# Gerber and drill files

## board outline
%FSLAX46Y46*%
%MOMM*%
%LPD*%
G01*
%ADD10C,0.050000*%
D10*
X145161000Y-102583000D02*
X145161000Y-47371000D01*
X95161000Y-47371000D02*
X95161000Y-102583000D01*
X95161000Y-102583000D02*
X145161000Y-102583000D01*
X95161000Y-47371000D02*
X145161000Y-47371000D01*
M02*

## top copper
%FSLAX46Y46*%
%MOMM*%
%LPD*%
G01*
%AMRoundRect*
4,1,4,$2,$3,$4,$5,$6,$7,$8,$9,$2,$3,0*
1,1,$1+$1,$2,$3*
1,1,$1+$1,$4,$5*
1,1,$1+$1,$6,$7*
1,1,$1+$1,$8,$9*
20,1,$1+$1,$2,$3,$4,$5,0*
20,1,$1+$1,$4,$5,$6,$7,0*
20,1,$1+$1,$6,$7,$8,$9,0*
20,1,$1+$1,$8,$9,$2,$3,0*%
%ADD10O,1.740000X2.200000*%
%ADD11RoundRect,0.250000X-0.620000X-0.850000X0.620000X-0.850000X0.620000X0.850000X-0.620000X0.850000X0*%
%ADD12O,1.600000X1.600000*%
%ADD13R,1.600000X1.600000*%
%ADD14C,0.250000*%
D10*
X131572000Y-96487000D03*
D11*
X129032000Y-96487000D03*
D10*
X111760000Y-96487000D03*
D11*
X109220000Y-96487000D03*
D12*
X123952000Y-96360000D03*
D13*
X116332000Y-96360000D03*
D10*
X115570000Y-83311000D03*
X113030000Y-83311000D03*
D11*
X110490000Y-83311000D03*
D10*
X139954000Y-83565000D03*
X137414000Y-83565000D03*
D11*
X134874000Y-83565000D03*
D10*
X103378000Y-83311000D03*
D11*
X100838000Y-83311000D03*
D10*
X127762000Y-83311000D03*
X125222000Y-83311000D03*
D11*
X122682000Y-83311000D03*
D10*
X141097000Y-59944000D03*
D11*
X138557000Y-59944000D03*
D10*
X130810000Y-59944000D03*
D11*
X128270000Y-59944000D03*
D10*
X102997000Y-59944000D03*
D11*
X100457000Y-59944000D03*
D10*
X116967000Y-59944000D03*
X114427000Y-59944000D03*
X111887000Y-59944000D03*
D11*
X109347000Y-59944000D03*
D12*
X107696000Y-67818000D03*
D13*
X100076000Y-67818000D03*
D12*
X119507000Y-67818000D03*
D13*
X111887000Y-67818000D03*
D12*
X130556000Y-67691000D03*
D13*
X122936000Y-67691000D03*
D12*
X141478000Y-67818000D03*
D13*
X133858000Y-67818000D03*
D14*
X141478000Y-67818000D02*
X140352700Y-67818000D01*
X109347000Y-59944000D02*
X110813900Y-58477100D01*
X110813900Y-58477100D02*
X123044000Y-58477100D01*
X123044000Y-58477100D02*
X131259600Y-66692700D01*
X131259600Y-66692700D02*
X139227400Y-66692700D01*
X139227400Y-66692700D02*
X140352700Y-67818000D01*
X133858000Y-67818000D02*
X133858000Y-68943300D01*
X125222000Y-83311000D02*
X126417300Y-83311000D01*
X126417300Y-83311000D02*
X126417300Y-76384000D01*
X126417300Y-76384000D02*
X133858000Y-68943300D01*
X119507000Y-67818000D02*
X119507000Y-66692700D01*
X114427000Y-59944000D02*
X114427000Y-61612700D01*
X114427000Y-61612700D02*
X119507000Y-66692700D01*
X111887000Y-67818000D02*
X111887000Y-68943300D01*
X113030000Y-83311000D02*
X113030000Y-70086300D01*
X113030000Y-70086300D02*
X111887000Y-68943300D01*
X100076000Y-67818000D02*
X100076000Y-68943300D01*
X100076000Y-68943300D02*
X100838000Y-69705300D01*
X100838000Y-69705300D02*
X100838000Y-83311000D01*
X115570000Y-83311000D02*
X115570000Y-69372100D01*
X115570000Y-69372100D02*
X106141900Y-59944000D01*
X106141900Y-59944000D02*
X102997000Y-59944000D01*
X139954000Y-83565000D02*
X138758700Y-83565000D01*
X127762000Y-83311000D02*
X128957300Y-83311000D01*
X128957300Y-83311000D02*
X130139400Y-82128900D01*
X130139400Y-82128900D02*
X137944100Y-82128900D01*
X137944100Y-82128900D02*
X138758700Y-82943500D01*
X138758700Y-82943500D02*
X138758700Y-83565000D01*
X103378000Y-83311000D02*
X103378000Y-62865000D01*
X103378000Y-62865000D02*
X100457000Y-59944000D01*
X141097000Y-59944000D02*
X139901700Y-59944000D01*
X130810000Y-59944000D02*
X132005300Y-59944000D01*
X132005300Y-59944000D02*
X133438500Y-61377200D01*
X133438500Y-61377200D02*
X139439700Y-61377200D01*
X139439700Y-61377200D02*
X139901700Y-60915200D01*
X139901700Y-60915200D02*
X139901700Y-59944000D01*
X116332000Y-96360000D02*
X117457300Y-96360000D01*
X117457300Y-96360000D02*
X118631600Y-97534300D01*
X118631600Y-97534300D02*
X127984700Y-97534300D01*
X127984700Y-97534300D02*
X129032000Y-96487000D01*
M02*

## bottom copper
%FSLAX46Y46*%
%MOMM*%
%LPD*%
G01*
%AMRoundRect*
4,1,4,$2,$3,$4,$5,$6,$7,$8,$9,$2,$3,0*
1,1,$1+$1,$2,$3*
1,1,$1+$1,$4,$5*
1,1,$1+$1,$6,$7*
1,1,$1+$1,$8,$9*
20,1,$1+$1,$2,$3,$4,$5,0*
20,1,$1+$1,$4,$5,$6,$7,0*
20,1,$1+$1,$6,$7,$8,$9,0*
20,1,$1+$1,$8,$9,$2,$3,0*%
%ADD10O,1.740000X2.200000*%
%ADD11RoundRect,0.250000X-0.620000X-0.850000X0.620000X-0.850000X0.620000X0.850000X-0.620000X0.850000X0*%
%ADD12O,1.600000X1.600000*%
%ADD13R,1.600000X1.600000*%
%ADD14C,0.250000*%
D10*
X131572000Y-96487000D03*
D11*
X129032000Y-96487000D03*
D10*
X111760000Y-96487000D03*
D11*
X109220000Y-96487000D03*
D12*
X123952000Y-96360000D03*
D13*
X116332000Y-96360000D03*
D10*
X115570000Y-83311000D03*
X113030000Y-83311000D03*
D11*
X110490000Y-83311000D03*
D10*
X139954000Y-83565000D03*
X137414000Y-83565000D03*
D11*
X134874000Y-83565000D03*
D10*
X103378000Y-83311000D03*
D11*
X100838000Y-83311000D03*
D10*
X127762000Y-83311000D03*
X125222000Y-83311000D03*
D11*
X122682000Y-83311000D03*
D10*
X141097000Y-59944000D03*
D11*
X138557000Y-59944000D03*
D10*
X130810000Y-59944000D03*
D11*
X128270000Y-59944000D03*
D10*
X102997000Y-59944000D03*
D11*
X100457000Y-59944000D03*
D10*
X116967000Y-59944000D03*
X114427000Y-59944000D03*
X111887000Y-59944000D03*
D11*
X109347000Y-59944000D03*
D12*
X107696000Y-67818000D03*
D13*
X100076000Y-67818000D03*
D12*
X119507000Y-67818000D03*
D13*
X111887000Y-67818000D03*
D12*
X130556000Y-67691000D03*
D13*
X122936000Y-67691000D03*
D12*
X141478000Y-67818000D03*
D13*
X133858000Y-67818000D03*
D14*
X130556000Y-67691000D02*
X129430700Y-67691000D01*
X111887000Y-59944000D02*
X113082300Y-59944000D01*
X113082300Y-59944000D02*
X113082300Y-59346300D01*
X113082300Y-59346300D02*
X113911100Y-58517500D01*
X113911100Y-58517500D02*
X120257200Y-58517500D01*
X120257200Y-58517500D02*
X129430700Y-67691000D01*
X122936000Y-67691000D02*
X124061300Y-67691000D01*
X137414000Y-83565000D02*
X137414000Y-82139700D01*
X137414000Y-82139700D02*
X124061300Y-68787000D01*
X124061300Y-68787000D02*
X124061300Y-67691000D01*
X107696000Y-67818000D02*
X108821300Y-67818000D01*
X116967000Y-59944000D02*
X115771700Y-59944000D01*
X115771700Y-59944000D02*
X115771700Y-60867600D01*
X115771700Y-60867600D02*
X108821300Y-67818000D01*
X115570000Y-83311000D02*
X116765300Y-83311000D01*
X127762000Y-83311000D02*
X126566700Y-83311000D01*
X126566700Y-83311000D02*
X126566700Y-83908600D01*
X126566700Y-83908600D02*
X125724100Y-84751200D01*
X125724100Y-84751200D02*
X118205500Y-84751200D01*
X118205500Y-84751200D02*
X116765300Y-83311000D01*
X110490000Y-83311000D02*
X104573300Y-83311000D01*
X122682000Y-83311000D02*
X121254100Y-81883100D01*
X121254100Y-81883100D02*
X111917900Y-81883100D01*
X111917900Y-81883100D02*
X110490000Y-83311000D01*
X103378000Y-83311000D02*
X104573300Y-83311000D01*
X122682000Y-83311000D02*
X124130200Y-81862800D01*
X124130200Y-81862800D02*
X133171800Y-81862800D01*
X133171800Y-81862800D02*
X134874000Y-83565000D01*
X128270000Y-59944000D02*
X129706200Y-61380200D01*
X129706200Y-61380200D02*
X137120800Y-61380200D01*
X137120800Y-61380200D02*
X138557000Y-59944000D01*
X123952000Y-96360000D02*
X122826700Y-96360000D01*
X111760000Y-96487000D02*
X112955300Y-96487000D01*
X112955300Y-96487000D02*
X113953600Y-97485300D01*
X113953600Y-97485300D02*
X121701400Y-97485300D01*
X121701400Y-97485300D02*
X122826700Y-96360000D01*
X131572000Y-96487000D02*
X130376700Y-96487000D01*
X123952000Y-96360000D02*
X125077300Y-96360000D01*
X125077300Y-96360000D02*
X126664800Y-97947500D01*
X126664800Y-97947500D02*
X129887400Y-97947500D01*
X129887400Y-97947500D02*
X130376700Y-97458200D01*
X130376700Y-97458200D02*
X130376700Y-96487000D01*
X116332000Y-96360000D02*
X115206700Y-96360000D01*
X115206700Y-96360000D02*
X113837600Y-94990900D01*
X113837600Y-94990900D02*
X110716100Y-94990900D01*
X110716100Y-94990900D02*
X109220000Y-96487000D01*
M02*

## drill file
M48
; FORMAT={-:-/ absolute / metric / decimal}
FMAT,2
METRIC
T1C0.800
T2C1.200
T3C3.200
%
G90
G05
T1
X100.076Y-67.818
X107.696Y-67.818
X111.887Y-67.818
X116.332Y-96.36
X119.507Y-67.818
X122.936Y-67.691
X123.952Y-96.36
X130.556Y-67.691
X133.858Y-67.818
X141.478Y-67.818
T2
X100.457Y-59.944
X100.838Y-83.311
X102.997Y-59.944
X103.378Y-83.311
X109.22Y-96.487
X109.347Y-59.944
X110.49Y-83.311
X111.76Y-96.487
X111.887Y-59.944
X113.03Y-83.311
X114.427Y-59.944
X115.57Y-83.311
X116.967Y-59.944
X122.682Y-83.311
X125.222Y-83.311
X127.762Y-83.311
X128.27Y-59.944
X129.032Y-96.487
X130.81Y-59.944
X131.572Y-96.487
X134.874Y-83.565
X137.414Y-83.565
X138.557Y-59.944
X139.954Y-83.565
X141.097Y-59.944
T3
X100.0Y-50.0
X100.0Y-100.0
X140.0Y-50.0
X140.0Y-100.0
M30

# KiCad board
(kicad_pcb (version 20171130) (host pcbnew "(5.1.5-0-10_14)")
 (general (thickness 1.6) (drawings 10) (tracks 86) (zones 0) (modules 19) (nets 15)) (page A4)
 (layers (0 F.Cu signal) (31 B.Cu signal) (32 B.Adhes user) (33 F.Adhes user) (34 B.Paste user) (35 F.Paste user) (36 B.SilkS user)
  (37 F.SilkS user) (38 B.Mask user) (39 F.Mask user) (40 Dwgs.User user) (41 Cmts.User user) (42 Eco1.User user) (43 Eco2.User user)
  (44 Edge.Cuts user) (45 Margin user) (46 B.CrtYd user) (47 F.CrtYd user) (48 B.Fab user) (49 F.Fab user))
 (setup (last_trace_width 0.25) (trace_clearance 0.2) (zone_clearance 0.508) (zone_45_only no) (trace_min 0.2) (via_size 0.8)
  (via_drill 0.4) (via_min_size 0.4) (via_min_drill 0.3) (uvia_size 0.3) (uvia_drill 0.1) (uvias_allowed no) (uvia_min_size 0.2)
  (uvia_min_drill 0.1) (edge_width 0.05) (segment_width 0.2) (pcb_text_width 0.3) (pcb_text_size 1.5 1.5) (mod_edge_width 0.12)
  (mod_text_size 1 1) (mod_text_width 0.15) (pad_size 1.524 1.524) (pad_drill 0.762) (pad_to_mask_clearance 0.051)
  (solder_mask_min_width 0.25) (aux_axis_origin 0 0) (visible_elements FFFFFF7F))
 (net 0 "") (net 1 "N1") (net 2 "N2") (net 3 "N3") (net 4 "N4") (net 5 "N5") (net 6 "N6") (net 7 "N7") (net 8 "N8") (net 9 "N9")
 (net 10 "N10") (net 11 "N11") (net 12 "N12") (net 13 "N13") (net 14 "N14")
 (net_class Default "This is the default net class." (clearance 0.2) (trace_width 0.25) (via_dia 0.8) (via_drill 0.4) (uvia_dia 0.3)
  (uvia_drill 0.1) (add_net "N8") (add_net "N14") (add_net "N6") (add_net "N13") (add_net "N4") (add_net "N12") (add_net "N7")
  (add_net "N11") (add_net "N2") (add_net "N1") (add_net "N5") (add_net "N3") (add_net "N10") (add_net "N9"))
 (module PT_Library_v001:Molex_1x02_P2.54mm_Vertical (layer F.Cu) (at 129.032 96.487)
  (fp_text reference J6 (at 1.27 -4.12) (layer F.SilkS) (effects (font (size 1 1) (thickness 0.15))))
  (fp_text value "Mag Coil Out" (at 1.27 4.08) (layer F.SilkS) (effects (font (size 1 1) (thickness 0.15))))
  (pad 2 thru_hole oval (at 2.54 0) (size 1.74 2.2) (drill 1.2) (layers *.Cu *.Mask) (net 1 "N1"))
  (pad 1 thru_hole roundrect (at 0 0) (size 1.74 2.2) (drill 1.2) (layers *.Cu *.Mask) (roundrect_rratio 0.143678) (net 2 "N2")))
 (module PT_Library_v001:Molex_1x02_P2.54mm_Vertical (layer F.Cu) (at 109.22 96.487)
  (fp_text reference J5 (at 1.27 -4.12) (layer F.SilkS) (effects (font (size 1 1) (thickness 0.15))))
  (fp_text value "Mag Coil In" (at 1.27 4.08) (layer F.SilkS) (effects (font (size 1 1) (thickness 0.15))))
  (pad 2 thru_hole oval (at 2.54 0) (size 1.74 2.2) (drill 1.2) (layers *.Cu *.Mask) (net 1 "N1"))
  (pad 1 thru_hole roundrect (at 0 0) (size 1.74 2.2) (drill 1.2) (layers *.Cu *.Mask) (roundrect_rratio 0.143678) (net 2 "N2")))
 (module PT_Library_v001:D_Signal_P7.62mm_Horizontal (layer F.Cu) (at 116.332 96.36)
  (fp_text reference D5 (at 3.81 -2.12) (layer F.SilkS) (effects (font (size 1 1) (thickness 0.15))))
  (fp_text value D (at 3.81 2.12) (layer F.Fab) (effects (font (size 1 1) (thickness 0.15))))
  (pad 2 thru_hole oval (at 7.62 0) (size 1.6 1.6) (drill 0.8) (layers *.Cu *.Mask) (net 1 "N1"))
  (pad 1 thru_hole rect (at 0 0) (size 1.6 1.6) (drill 0.8) (layers *.Cu *.Mask) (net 2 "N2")))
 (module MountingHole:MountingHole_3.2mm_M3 (layer F.Cu) (at 140 100)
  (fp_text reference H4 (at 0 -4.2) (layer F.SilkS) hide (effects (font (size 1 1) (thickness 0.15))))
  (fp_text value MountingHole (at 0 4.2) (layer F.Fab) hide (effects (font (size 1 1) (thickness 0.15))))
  (pad 1 np_thru_hole circle (at 0 0) (size 3.2 3.2) (drill 3.2) (layers *.Cu *.Mask)))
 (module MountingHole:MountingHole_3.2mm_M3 (layer F.Cu) (at 100 100)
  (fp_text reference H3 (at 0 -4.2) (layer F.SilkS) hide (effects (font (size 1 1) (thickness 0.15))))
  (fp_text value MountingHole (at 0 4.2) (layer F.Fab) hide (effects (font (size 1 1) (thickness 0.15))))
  (pad 1 np_thru_hole circle (at 0 0) (size 3.2 3.2) (drill 3.2) (layers *.Cu *.Mask)))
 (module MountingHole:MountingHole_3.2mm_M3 (layer F.Cu) (at 140 50)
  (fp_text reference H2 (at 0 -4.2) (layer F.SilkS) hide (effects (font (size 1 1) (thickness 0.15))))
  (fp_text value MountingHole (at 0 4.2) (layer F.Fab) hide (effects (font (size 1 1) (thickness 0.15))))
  (pad 1 np_thru_hole circle (at 0 0) (size 3.2 3.2) (drill 3.2) (layers *.Cu *.Mask)))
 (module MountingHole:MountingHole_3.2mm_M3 (layer F.Cu) (at 100 50)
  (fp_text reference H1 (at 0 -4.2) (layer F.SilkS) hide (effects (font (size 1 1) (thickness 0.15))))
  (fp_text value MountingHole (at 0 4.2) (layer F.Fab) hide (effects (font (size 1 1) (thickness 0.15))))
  (pad 1 np_thru_hole circle (at 0 0) (size 3.2 3.2) (drill 3.2) (layers *.Cu *.Mask)))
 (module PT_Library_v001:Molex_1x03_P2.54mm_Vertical (layer F.Cu) (at 110.49 83.311)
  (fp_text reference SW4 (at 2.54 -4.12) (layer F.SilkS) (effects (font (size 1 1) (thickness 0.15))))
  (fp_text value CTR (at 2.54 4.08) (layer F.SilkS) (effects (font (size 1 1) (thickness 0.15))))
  (pad 3 thru_hole oval (at 5.08 0) (size 1.74 2.2) (drill 1.2) (layers *.Cu *.Mask) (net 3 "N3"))
  (pad 2 thru_hole oval (at 2.54 0) (size 1.74 2.2) (drill 1.2) (layers *.Cu *.Mask) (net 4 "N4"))
  (pad 1 thru_hole roundrect (at 0 0) (size 1.74 2.2) (drill 1.2) (layers *.Cu *.Mask) (roundrect_rratio 0.143678) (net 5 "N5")))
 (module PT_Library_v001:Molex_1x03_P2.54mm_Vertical (layer F.Cu) (at 134.874 83.565)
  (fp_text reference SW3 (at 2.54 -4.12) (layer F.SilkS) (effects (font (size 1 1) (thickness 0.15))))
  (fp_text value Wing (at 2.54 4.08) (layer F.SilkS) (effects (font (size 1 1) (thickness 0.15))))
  (pad 3 thru_hole oval (at 5.08 0) (size 1.74 2.2) (drill 1.2) (layers *.Cu *.Mask) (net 3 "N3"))
  (pad 2 thru_hole oval (at 2.54 0) (size 1.74 2.2) (drill 1.2) (layers *.Cu *.Mask) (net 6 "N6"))
  (pad 1 thru_hole roundrect (at 0 0) (size 1.74 2.2) (drill 1.2) (layers *.Cu *.Mask) (roundrect_rratio 0.143678) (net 5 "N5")))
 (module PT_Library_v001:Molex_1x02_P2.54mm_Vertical (layer F.Cu) (at 100.838 83.311)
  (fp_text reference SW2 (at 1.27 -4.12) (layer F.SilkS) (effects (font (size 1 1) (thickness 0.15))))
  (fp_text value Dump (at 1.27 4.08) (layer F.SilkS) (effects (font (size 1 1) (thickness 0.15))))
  (pad 2 thru_hole oval (at 2.54 0) (size 1.74 2.2) (drill 1.2) (layers *.Cu *.Mask) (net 5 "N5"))
  (pad 1 thru_hole roundrect (at 0 0) (size 1.74 2.2) (drill 1.2) (layers *.Cu *.Mask) (roundrect_rratio 0.143678) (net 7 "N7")))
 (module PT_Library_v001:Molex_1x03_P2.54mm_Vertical (layer F.Cu) (at 122.682 83.311)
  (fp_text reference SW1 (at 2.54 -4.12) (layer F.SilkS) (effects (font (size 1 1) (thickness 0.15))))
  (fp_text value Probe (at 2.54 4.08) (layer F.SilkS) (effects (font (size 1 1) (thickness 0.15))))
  (pad 3 thru_hole oval (at 5.08 0) (size 1.74 2.2) (drill 1.2) (layers *.Cu *.Mask) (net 3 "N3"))
  (pad 2 thru_hole oval (at 2.54 0) (size 1.74 2.2) (drill 1.2) (layers *.Cu *.Mask) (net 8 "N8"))
  (pad 1 thru_hole roundrect (at 0 0) (size 1.74 2.2) (drill 1.2) (layers *.Cu *.Mask) (roundrect_rratio 0.143678) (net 5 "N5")))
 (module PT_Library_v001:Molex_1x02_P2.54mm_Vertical (layer F.Cu) (at 138.557 59.944)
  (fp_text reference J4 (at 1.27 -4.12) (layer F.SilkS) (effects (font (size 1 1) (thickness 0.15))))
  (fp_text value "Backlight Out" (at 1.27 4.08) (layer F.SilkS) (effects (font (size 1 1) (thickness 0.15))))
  (pad 2 thru_hole oval (at 2.54 0) (size 1.74 2.2) (drill 1.2) (layers *.Cu *.Mask) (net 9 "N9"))
  (pad 1 thru_hole roundrect (at 0 0) (size 1.74 2.2) (drill 1.2) (layers *.Cu *.Mask) (roundrect_rratio 0.143678) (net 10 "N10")))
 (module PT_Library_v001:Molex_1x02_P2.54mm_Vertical (layer F.Cu) (at 128.27 59.944)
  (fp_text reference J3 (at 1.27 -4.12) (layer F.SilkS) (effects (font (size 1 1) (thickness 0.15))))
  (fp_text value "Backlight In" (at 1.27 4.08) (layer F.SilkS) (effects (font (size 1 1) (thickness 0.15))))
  (pad 2 thru_hole oval (at 2.54 0) (size 1.74 2.2) (drill 1.2) (layers *.Cu *.Mask) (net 9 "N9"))
  (pad 1 thru_hole roundrect (at 0 0) (size 1.74 2.2) (drill 1.2) (layers *.Cu *.Mask) (roundrect_rratio 0.143678) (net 10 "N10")))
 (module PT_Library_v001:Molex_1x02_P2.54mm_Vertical (layer F.Cu) (at 100.457 59.944)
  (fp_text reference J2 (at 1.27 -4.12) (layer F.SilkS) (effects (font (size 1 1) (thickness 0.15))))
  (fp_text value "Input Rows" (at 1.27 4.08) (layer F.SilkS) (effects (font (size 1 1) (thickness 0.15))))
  (pad 2 thru_hole oval (at 2.54 0) (size 1.74 2.2) (drill 1.2) (layers *.Cu *.Mask) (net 3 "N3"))
  (pad 1 thru_hole roundrect (at 0 0) (size 1.74 2.2) (drill 1.2) (layers *.Cu *.Mask) (roundrect_rratio 0.143678) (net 5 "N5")))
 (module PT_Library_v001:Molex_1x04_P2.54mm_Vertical (layer F.Cu) (at 109.347 59.944)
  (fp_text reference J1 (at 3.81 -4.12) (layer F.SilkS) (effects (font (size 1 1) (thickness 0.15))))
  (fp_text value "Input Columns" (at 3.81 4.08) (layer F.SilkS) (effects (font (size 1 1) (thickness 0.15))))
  (pad 4 thru_hole oval (at 7.62 0) (size 1.74 2.2) (drill 1.2) (layers *.Cu *.Mask) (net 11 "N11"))
  (pad 3 thru_hole oval (at 5.08 0) (size 1.74 2.2) (drill 1.2) (layers *.Cu *.Mask) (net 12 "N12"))
  (pad 2 thru_hole oval (at 2.54 0) (size 1.74 2.2) (drill 1.2) (layers *.Cu *.Mask) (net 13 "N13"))
  (pad 1 thru_hole roundrect (at 0 0) (size 1.74 2.2) (drill 1.2) (layers *.Cu *.Mask) (roundrect_rratio 0.143678) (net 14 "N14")))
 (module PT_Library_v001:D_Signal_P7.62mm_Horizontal (layer F.Cu) (at 100.076 67.818)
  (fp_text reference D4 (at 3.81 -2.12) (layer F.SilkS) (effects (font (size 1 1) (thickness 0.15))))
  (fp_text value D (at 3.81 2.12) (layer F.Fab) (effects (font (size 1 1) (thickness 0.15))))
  (pad 2 thru_hole oval (at 7.62 0) (size 1.6 1.6) (drill 0.8) (layers *.Cu *.Mask) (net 11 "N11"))
  (pad 1 thru_hole rect (at 0 0) (size 1.6 1.6) (drill 0.8) (layers *.Cu *.Mask) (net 7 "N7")))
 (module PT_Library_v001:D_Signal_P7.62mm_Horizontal (layer F.Cu) (at 111.887 67.818)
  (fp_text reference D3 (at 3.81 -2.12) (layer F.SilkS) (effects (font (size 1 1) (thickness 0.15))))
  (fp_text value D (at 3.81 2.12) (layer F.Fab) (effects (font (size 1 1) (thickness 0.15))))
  (pad 2 thru_hole oval (at 7.62 0) (size 1.6 1.6) (drill 0.8) (layers *.Cu *.Mask) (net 12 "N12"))
  (pad 1 thru_hole rect (at 0 0) (size 1.6 1.6) (drill 0.8) (layers *.Cu *.Mask) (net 4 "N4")))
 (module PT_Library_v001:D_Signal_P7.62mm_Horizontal (layer F.Cu) (at 122.936 67.691)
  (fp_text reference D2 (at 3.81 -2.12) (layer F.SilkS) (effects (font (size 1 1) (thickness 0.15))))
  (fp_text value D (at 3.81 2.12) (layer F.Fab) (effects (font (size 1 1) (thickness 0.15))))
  (pad 2 thru_hole oval (at 7.62 0) (size 1.6 1.6) (drill 0.8) (layers *.Cu *.Mask) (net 13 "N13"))
  (pad 1 thru_hole rect (at 0 0) (size 1.6 1.6) (drill 0.8) (layers *.Cu *.Mask) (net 6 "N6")))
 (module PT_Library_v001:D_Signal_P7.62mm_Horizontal (layer F.Cu) (at 133.858 67.818)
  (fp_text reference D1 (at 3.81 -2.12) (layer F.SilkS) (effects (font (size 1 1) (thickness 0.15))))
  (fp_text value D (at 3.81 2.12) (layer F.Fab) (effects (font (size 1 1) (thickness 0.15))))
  (pad 2 thru_hole oval (at 7.62 0) (size 1.6 1.6) (drill 0.8) (layers *.Cu *.Mask) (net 14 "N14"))
  (pad 1 thru_hole rect (at 0 0) (size 1.6 1.6) (drill 0.8) (layers *.Cu *.Mask) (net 8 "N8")))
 (gr_line (start 145.161 102.583) (end 145.161 47.371) (layer Edge.Cuts) (width 0.05))
 (gr_line (start 95.161 47.371) (end 95.161 102.583) (layer Edge.Cuts) (width 0.05))
 (gr_line (start 95.161 102.583) (end 145.161 102.583) (layer Edge.Cuts) (width 0.05))
 (gr_line (start 95.161 47.371) (end 145.161 47.371) (layer Edge.Cuts) (width 0.05))
 (segment (start 141.478 67.818) (end 140.3527 67.818) (width 0.25) (layer F.Cu) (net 14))
 (segment (start 109.347 59.944) (end 110.8139 58.4771) (width 0.25) (layer F.Cu) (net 14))
 (segment (start 110.8139 58.4771) (end 123.044 58.4771) (width 0.25) (layer F.Cu) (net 14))
 (segment (start 123.044 58.4771) (end 131.2596 66.6927) (width 0.25) (layer F.Cu) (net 14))
 (segment (start 131.2596 66.6927) (end 139.2274 66.6927) (width 0.25) (layer F.Cu) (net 14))
 (segment (start 139.2274 66.6927) (end 140.3527 67.818) (width 0.25) (layer F.Cu) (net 14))
 (segment (start 133.858 67.818) (end 133.858 68.9433) (width 0.25) (layer F.Cu) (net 8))
 (segment (start 125.222 83.311) (end 126.4173 83.311) (width 0.25) (layer F.Cu) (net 8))
 (segment (start 126.4173 83.311) (end 126.4173 76.384) (width 0.25) (layer F.Cu) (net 8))
 (segment (start 126.4173 76.384) (end 133.858 68.9433) (width 0.25) (layer F.Cu) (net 8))
 (segment (start 130.556 67.691) (end 129.4307 67.691) (width 0.25) (layer B.Cu) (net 13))
 (segment (start 111.887 59.944) (end 113.0823 59.944) (width 0.25) (layer B.Cu) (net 13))
 (segment (start 113.0823 59.944) (end 113.0823 59.3463) (width 0.25) (layer B.Cu) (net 13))
 (segment (start 113.0823 59.3463) (end 113.9111 58.5175) (width 0.25) (layer B.Cu) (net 13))
 (segment (start 113.9111 58.5175) (end 120.2572 58.5175) (width 0.25) (layer B.Cu) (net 13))
 (segment (start 120.2572 58.5175) (end 129.4307 67.691) (width 0.25) (layer B.Cu) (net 13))
 (segment (start 122.936 67.691) (end 124.0613 67.691) (width 0.25) (layer B.Cu) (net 6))
 (segment (start 137.414 83.565) (end 137.414 82.1397) (width 0.25) (layer B.Cu) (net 6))
 (segment (start 137.414 82.1397) (end 124.0613 68.787) (width 0.25) (layer B.Cu) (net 6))
 (segment (start 124.0613 68.787) (end 124.0613 67.691) (width 0.25) (layer B.Cu) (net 6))
 (segment (start 119.507 67.818) (end 119.507 66.6927) (width 0.25) (layer F.Cu) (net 12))
 (segment (start 114.427 59.944) (end 114.427 61.6127) (width 0.25) (layer F.Cu) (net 12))
 (segment (start 114.427 61.6127) (end 119.507 66.6927) (width 0.25) (layer F.Cu) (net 12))
 (segment (start 111.887 67.818) (end 111.887 68.9433) (width 0.25) (layer F.Cu) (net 4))
 (segment (start 113.03 83.311) (end 113.03 70.0863) (width 0.25) (layer F.Cu) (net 4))
 (segment (start 113.03 70.0863) (end 111.887 68.9433) (width 0.25) (layer F.Cu) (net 4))
 (segment (start 107.696 67.818) (end 108.8213 67.818) (width 0.25) (layer B.Cu) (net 11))
 (segment (start 116.967 59.944) (end 115.7717 59.944) (width 0.25) (layer B.Cu) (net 11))
 (segment (start 115.7717 59.944) (end 115.7717 60.8676) (width 0.25) (layer B.Cu) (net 11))
 (segment (start 115.7717 60.8676) (end 108.8213 67.818) (width 0.25) (layer B.Cu) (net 11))
 (segment (start 100.076 67.818) (end 100.076 68.9433) (width 0.25) (layer F.Cu) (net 7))
 (segment (start 100.076 68.9433) (end 100.838 69.7053) (width 0.25) (layer F.Cu) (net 7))
 (segment (start 100.838 69.7053) (end 100.838 83.311) (width 0.25) (layer F.Cu) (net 7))
 (segment (start 115.57 83.311) (end 115.57 69.3721) (width 0.25) (layer F.Cu) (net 3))
 (segment (start 115.57 69.3721) (end 106.1419 59.944) (width 0.25) (layer F.Cu) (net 3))
 (segment (start 106.1419 59.944) (end 102.997 59.944) (width 0.25) (layer F.Cu) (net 3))
 (segment (start 115.57 83.311) (end 116.7653 83.311) (width 0.25) (layer B.Cu) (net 3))
 (segment (start 127.762 83.311) (end 126.5667 83.311) (width 0.25) (layer B.Cu) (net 3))
 (segment (start 126.5667 83.311) (end 126.5667 83.9086) (width 0.25) (layer B.Cu) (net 3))
 (segment (start 126.5667 83.9086) (end 125.7241 84.7512) (width 0.25) (layer B.Cu) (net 3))
 (segment (start 125.7241 84.7512) (end 118.2055 84.7512) (width 0.25) (layer B.Cu) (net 3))
 (segment (start 118.2055 84.7512) (end 116.7653 83.311) (width 0.25) (layer B.Cu) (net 3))
 (segment (start 139.954 83.565) (end 138.7587 83.565) (width 0.25) (layer F.Cu) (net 3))
 (segment (start 127.762 83.311) (end 128.9573 83.311) (width 0.25) (layer F.Cu) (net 3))
 (segment (start 128.9573 83.311) (end 130.1394 82.1289) (width 0.25) (layer F.Cu) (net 3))
 (segment (start 130.1394 82.1289) (end 137.9441 82.1289) (width 0.25) (layer F.Cu) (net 3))
 (segment (start 137.9441 82.1289) (end 138.7587 82.9435) (width 0.25) (layer F.Cu) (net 3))
 (segment (start 138.7587 82.9435) (end 138.7587 83.565) (width 0.25) (layer F.Cu) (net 3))
 (segment (start 103.378 83.311) (end 103.378 62.865) (width 0.25) (layer F.Cu) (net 5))
 (segment (start 103.378 62.865) (end 100.457 59.944) (width 0.25) (layer F.Cu) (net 5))
 (segment (start 110.49 83.311) (end 104.5733 83.311) (width 0.25) (layer B.Cu) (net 5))
 (segment (start 122.682 83.311) (end 121.2541 81.8831) (width 0.25) (layer B.Cu) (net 5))
 (segment (start 121.2541 81.8831) (end 111.9179 81.8831) (width 0.25) (layer B.Cu) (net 5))
 (segment (start 111.9179 81.8831) (end 110.49 83.311) (width 0.25) (layer B.Cu) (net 5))
 (segment (start 103.378 83.311) (end 104.5733 83.311) (width 0.25) (layer B.Cu) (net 5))
 (segment (start 122.682 83.311) (end 124.1302 81.8628) (width 0.25) (layer B.Cu) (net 5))
 (segment (start 124.1302 81.8628) (end 133.1718 81.8628) (width 0.25) (layer B.Cu) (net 5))
 (segment (start 133.1718 81.8628) (end 134.874 83.565) (width 0.25) (layer B.Cu) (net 5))
 (segment (start 141.097 59.944) (end 139.9017 59.944) (width 0.25) (layer F.Cu) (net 9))
 (segment (start 130.81 59.944) (end 132.0053 59.944) (width 0.25) (layer F.Cu) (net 9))
 (segment (start 132.0053 59.944) (end 133.4385 61.3772) (width 0.25) (layer F.Cu) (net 9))
 (segment (start 133.4385 61.3772) (end 139.4397 61.3772) (width 0.25) (layer F.Cu) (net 9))
 (segment (start 139.4397 61.3772) (end 139.9017 60.9152) (width 0.25) (layer F.Cu) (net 9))
 (segment (start 139.9017 60.9152) (end 139.9017 59.944) (width 0.25) (layer F.Cu) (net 9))
 (segment (start 128.27 59.944) (end 129.7062 61.3802) (width 0.25) (layer B.Cu) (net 10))
 (segment (start 129.7062 61.3802) (end 137.1208 61.3802) (width 0.25) (layer B.Cu) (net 10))
 (segment (start 137.1208 61.3802) (end 138.557 59.944) (width 0.25) (layer B.Cu) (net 10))
 (segment (start 123.952 96.36) (end 122.8267 96.36) (width 0.25) (layer B.Cu) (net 1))
 (segment (start 111.76 96.487) (end 112.9553 96.487) (width 0.25) (layer B.Cu) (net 1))
 (segment (start 112.9553 96.487) (end 113.9536 97.4853) (width 0.25) (layer B.Cu) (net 1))
 (segment (start 113.9536 97.4853) (end 121.7014 97.4853) (width 0.25) (layer B.Cu) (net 1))
 (segment (start 121.7014 97.4853) (end 122.8267 96.36) (width 0.25) (layer B.Cu) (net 1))
 (segment (start 131.572 96.487) (end 130.3767 96.487) (width 0.25) (layer B.Cu) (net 1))
 (segment (start 123.952 96.36) (end 125.0773 96.36) (width 0.25) (layer B.Cu) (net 1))
 (segment (start 125.0773 96.36) (end 126.6648 97.9475) (width 0.25) (layer B.Cu) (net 1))
 (segment (start 126.6648 97.9475) (end 129.8874 97.9475) (width 0.25) (layer B.Cu) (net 1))
 (segment (start 129.8874 97.9475) (end 130.3767 97.4582) (width 0.25) (layer B.Cu) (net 1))
 (segment (start 130.3767 97.4582) (end 130.3767 96.487) (width 0.25) (layer B.Cu) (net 1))
 (segment (start 116.332 96.36) (end 117.4573 96.36) (width 0.25) (layer F.Cu) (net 2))
 (segment (start 117.4573 96.36) (end 118.6316 97.5343) (width 0.25) (layer F.Cu) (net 2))
 (segment (start 118.6316 97.5343) (end 127.9847 97.5343) (width 0.25) (layer F.Cu) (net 2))
 (segment (start 127.9847 97.5343) (end 129.032 96.487) (width 0.25) (layer F.Cu) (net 2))
 (segment (start 116.332 96.36) (end 115.2067 96.36) (width 0.25) (layer B.Cu) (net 2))
 (segment (start 115.2067 96.36) (end 113.8376 94.9909) (width 0.25) (layer B.Cu) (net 2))
 (segment (start 113.8376 94.9909) (end 110.7161 94.9909) (width 0.25) (layer B.Cu) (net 2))
 (segment (start 110.7161 94.9909) (end 109.22 96.487) (width 0.25) (layer B.Cu) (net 2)))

